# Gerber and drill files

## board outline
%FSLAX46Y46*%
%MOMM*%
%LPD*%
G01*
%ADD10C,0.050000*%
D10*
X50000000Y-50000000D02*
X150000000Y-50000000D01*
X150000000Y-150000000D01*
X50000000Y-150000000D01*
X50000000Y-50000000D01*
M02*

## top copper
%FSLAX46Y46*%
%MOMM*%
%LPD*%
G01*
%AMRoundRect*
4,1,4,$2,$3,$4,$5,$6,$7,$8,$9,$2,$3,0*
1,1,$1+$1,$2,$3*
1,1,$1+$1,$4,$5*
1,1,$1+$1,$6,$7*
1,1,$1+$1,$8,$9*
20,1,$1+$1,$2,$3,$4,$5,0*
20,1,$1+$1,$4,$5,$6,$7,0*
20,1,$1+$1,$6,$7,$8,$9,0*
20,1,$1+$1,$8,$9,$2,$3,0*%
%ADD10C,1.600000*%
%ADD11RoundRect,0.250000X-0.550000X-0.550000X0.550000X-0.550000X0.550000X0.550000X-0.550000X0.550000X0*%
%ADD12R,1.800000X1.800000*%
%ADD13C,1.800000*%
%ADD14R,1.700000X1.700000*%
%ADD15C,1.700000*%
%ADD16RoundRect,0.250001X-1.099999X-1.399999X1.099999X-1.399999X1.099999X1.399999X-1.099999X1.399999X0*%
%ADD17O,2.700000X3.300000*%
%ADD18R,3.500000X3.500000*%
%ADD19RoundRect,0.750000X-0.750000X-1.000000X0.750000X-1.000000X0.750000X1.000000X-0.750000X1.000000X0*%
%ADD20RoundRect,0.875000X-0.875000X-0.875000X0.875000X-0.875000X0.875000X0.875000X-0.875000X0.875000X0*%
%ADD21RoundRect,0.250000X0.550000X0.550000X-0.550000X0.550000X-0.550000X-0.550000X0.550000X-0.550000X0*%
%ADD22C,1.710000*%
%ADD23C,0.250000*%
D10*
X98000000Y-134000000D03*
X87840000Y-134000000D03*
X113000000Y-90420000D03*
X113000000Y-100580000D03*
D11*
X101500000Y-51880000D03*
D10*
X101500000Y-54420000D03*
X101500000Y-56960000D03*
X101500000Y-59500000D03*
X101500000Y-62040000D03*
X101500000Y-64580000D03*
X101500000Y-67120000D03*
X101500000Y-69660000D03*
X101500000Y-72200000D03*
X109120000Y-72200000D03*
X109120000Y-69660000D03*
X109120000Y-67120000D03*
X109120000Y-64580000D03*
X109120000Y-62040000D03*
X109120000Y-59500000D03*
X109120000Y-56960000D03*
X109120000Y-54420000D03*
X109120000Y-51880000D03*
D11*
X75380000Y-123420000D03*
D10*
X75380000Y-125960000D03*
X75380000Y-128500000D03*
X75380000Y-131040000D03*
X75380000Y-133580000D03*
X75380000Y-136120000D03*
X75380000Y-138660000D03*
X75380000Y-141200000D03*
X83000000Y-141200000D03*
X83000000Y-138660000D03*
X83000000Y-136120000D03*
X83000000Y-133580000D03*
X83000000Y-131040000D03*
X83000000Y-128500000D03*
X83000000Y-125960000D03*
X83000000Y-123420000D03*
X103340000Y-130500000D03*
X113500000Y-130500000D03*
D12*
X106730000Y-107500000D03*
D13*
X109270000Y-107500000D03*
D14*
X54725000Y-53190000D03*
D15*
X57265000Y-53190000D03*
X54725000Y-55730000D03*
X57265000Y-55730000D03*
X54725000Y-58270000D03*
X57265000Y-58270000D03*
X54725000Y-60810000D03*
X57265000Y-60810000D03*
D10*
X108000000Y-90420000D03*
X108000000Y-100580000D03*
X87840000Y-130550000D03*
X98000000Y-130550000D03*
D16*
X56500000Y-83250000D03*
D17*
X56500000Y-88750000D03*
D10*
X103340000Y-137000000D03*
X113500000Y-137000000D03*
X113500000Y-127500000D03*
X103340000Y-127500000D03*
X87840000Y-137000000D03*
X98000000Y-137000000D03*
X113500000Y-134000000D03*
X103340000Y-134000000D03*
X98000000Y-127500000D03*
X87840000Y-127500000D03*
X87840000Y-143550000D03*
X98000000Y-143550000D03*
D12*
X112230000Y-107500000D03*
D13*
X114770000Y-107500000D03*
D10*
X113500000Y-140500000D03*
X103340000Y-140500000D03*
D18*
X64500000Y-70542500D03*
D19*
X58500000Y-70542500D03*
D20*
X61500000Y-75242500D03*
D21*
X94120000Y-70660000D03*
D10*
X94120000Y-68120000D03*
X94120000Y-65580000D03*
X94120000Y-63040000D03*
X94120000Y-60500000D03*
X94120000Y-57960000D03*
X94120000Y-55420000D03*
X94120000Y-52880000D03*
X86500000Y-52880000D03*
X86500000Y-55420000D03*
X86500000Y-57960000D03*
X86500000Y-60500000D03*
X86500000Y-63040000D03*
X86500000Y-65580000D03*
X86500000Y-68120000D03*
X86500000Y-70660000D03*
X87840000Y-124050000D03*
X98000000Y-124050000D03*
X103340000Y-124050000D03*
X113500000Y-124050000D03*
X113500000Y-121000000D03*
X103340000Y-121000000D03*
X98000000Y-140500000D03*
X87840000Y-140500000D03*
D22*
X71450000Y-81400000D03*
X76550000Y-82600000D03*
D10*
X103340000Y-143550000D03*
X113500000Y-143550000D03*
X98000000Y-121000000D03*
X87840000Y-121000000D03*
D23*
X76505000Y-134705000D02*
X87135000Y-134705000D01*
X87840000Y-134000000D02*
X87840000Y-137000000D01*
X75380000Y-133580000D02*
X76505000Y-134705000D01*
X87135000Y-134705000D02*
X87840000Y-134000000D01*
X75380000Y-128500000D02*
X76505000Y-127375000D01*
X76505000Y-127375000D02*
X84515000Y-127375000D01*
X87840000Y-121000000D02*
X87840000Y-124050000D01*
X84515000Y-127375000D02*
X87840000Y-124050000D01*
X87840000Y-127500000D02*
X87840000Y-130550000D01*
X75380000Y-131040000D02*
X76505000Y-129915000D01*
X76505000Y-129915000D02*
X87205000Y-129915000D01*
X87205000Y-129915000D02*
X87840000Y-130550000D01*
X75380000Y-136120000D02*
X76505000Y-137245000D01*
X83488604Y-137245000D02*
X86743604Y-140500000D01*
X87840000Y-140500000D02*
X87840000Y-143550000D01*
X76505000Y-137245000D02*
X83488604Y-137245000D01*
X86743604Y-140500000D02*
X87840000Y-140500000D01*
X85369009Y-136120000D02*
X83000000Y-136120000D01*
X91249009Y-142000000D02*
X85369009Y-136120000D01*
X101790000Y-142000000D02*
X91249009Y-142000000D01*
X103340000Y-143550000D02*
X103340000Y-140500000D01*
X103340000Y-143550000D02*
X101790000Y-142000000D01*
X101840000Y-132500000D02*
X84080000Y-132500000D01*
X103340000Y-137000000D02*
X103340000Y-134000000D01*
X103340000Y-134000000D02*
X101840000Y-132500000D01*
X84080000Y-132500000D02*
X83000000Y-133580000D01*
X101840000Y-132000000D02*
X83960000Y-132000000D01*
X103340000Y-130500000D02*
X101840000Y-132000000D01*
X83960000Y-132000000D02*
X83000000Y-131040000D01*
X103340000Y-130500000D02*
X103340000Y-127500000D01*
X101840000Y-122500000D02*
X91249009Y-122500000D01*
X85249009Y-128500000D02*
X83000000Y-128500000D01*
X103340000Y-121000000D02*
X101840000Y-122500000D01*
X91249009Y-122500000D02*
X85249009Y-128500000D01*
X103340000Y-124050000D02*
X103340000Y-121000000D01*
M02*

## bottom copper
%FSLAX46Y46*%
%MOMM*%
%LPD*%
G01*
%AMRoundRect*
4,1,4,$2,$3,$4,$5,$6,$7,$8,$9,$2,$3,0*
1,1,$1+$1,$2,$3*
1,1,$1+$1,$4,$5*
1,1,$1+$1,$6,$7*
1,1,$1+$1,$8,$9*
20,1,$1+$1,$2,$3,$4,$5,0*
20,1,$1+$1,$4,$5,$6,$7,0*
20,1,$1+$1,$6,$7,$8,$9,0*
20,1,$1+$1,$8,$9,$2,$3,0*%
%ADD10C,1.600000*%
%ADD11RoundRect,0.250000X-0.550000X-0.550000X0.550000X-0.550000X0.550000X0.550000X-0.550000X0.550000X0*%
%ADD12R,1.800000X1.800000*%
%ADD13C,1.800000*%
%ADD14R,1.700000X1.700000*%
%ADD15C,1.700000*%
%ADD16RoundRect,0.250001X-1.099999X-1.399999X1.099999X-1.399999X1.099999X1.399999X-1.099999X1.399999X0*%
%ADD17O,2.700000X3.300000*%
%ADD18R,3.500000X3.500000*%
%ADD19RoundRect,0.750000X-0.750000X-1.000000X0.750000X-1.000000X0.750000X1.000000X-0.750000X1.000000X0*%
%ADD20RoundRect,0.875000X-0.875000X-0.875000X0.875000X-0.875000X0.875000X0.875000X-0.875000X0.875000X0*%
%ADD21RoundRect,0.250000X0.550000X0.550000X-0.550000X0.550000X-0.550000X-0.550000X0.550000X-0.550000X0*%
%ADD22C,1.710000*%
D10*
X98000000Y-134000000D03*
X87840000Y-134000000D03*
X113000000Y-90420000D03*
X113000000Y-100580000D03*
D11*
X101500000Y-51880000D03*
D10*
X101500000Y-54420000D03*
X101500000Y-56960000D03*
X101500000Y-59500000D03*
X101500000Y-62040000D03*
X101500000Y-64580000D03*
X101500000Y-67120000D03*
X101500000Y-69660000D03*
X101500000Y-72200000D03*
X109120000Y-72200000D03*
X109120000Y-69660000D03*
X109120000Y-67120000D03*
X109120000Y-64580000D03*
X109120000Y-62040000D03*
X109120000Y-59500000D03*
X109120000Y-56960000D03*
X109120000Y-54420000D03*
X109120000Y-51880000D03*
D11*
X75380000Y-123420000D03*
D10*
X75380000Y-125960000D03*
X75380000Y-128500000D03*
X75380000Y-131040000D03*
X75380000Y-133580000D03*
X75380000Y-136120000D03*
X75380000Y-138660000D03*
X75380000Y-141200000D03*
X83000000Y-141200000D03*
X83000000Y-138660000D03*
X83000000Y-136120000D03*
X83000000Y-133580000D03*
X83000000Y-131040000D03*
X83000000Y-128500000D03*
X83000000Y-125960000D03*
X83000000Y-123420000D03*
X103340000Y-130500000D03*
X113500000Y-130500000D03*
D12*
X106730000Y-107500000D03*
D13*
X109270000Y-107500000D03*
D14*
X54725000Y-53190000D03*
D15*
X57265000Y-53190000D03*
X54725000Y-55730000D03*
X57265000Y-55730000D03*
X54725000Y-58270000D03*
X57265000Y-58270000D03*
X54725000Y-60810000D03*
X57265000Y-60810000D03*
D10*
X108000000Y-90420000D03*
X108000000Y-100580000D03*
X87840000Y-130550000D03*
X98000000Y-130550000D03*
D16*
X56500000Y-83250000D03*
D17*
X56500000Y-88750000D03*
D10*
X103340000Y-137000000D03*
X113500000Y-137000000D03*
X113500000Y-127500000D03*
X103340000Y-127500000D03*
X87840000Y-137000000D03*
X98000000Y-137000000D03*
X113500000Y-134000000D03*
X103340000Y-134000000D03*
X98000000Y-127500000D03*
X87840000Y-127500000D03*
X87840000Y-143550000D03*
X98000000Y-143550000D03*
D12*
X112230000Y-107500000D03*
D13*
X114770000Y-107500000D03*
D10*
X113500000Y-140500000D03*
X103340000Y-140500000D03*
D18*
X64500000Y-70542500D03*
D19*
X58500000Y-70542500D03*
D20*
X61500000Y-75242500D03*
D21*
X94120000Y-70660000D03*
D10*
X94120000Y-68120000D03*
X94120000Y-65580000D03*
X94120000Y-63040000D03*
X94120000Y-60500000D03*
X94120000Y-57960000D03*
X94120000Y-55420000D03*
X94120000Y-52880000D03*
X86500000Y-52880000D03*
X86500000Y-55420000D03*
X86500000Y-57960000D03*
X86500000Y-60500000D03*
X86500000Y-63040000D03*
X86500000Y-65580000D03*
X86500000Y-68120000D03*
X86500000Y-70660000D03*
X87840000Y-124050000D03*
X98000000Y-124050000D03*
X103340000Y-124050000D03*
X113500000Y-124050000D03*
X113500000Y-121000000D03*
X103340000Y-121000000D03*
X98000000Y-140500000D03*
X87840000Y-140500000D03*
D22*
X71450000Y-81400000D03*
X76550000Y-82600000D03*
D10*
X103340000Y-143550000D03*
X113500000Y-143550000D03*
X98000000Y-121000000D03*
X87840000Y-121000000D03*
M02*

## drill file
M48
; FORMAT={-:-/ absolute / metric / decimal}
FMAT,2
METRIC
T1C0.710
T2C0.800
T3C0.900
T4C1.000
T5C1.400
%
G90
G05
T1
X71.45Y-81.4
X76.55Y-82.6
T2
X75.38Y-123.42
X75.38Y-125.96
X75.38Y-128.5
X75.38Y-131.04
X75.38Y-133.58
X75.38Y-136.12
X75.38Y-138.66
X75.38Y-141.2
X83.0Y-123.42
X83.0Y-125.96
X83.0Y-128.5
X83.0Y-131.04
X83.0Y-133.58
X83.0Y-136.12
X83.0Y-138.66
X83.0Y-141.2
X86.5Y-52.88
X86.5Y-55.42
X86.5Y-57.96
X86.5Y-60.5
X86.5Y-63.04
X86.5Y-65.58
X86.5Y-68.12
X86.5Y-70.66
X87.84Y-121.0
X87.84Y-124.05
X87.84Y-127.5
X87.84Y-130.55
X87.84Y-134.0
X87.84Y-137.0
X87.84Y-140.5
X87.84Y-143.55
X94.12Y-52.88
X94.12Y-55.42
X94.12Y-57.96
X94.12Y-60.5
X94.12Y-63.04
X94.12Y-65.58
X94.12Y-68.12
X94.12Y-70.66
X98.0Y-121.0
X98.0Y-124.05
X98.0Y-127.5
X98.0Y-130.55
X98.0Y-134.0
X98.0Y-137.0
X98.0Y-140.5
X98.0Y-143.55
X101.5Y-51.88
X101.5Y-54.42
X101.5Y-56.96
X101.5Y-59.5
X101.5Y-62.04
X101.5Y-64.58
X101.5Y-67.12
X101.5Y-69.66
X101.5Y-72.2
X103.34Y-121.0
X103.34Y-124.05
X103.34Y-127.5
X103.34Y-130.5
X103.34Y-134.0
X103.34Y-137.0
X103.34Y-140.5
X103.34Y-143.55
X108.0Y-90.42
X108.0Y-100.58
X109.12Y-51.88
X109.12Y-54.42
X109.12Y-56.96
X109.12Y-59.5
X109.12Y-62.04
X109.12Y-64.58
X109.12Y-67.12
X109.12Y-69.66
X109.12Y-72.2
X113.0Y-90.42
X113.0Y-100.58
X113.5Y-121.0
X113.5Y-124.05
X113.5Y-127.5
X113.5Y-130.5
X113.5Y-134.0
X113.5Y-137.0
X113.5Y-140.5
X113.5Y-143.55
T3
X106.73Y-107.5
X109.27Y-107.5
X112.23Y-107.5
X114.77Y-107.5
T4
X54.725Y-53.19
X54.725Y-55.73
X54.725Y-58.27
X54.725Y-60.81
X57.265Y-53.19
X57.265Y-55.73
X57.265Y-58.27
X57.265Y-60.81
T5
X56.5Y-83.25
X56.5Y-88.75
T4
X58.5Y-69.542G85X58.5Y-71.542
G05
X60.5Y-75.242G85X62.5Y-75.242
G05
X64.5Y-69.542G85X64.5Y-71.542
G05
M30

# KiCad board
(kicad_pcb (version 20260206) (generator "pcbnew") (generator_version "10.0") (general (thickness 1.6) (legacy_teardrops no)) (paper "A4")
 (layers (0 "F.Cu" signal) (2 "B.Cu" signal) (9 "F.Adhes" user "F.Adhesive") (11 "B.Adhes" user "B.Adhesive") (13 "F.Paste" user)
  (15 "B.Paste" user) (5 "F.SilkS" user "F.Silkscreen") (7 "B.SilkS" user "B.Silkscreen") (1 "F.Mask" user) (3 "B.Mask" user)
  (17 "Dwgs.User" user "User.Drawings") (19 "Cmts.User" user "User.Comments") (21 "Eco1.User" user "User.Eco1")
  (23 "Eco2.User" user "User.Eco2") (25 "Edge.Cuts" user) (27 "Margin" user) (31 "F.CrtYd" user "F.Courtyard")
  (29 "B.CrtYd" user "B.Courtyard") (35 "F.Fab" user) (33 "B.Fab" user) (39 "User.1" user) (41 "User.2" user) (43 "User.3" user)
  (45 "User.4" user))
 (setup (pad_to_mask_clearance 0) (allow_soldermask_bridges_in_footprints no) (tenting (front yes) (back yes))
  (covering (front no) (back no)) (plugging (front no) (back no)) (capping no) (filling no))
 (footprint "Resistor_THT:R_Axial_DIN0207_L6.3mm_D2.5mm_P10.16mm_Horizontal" (layer "F.Cu") (at 98 134 180)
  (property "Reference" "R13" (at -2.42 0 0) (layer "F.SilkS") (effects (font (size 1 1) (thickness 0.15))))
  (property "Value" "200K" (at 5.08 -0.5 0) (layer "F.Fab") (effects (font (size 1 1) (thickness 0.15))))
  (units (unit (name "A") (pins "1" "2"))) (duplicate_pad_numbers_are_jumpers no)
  (pad "1" thru_hole circle (at 0 0 180) (size 1.6 1.6) (drill 0.8) (layers "*.Cu" "*.Mask") (remove_unused_layers no) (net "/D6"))
  (pad "2" thru_hole circle (at 10.16 0 180) (size 1.6 1.6) (drill 0.8) (layers "*.Cu" "*.Mask") (remove_unused_layers no)
   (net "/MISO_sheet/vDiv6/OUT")))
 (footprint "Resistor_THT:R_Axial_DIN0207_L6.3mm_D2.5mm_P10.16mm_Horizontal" (layer "F.Cu") (at 113 90.42 -90)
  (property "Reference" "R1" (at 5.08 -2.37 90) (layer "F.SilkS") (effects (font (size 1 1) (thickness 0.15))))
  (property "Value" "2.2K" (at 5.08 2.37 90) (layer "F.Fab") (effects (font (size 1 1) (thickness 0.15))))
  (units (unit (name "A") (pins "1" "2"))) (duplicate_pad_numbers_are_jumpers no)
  (pad "1" thru_hole circle (at 0 0 270) (size 1.6 1.6) (drill 0.8) (layers "*.Cu" "*.Mask") (remove_unused_layers no) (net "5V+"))
  (pad "2" thru_hole circle (at 10.16 0 270) (size 1.6 1.6) (drill 0.8) (layers "*.Cu" "*.Mask") (remove_unused_layers no)
   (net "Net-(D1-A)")))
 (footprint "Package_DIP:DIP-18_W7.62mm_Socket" (layer "F.Cu") (at 101.5 51.88)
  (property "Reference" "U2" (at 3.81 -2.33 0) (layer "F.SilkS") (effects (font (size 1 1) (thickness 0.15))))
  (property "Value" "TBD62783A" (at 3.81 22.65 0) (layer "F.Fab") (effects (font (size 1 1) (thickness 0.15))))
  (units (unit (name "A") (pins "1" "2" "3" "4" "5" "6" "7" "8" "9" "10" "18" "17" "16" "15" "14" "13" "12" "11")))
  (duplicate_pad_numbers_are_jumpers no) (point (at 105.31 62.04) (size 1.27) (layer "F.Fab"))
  (pad "1" thru_hole roundrect (at 0 0) (size 1.6 1.6) (drill 0.8) (layers "*.Cu" "*.Mask") (remove_unused_layers no)
   (roundrect_rratio 0.15625) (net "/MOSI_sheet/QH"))
  (pad "2" thru_hole circle (at 0 2.54) (size 1.6 1.6) (drill 0.8) (layers "*.Cu" "*.Mask") (remove_unused_layers no) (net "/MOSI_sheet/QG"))
  (pad "3" thru_hole circle (at 0 5.08) (size 1.6 1.6) (drill 0.8) (layers "*.Cu" "*.Mask") (remove_unused_layers no) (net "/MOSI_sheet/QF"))
  (pad "4" thru_hole circle (at 0 7.62) (size 1.6 1.6) (drill 0.8) (layers "*.Cu" "*.Mask") (remove_unused_layers no) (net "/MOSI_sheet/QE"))
  (pad "5" thru_hole circle (at 0 10.16) (size 1.6 1.6) (drill 0.8) (layers "*.Cu" "*.Mask") (remove_unused_layers no)
   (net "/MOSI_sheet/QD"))
  (pad "6" thru_hole circle (at 0 12.7) (size 1.6 1.6) (drill 0.8) (layers "*.Cu" "*.Mask") (remove_unused_layers no) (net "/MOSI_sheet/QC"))
  (pad "7" thru_hole circle (at 0 15.24) (size 1.6 1.6) (drill 0.8) (layers "*.Cu" "*.Mask") (remove_unused_layers no)
   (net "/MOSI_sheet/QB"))
  (pad "8" thru_hole circle (at 0 17.78) (size 1.6 1.6) (drill 0.8) (layers "*.Cu" "*.Mask") (remove_unused_layers no)
   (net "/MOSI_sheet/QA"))
  (pad "9" thru_hole circle (at 0 20.32) (size 1.6 1.6) (drill 0.8) (layers "*.Cu" "*.Mask") (remove_unused_layers no) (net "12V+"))
  (pad "10" thru_hole circle (at 7.62 20.32) (size 1.6 1.6) (drill 0.8) (layers "*.Cu" "*.Mask") (remove_unused_layers no) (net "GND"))
  (pad "11" thru_hole circle (at 7.62 17.78) (size 1.6 1.6) (drill 0.8) (layers "*.Cu" "*.Mask") (remove_unused_layers no)
   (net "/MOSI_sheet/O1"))
  (pad "12" thru_hole circle (at 7.62 15.24) (size 1.6 1.6) (drill 0.8) (layers "*.Cu" "*.Mask") (remove_unused_layers no)
   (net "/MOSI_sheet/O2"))
  (pad "13" thru_hole circle (at 7.62 12.7) (size 1.6 1.6) (drill 0.8) (layers "*.Cu" "*.Mask") (remove_unused_layers no)
   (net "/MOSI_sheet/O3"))
  (pad "14" thru_hole circle (at 7.62 10.16) (size 1.6 1.6) (drill 0.8) (layers "*.Cu" "*.Mask") (remove_unused_layers no)
   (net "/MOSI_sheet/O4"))
  (pad "15" thru_hole circle (at 7.62 7.62) (size 1.6 1.6) (drill 0.8) (layers "*.Cu" "*.Mask") (remove_unused_layers no)
   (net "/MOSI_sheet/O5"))
  (pad "16" thru_hole circle (at 7.62 5.08) (size 1.6 1.6) (drill 0.8) (layers "*.Cu" "*.Mask") (remove_unused_layers no)
   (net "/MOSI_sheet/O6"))
  (pad "17" thru_hole circle (at 7.62 2.54) (size 1.6 1.6) (drill 0.8) (layers "*.Cu" "*.Mask") (remove_unused_layers no)
   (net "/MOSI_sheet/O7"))
  (pad "18" thru_hole circle (at 7.62 0) (size 1.6 1.6) (drill 0.8) (layers "*.Cu" "*.Mask") (remove_unused_layers no)
   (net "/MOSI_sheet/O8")))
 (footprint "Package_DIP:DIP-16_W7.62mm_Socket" (layer "F.Cu") (at 75.38 123.42)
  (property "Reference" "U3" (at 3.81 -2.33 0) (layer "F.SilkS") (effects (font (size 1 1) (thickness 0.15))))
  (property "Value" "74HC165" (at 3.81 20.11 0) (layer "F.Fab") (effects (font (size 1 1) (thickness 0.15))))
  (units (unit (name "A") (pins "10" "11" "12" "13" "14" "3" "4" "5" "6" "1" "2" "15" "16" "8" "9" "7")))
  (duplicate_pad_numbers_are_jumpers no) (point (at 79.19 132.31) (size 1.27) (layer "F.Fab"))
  (pad "1" thru_hole roundrect (at 0 0) (size 1.6 1.6) (drill 0.8) (layers "*.Cu" "*.Mask") (remove_unused_layers no)
   (roundrect_rratio 0.15625) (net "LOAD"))
  (pad "2" thru_hole circle (at 0 2.54) (size 1.6 1.6) (drill 0.8) (layers "*.Cu" "*.Mask") (remove_unused_layers no) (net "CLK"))
  (pad "3" thru_hole circle (at 0 5.08) (size 1.6 1.6) (drill 0.8) (layers "*.Cu" "*.Mask") (remove_unused_layers no)
   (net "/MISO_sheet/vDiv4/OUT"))
  (pad "4" thru_hole circle (at 0 7.62) (size 1.6 1.6) (drill 0.8) (layers "*.Cu" "*.Mask") (remove_unused_layers no)
   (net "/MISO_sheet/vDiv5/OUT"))
  (pad "5" thru_hole circle (at 0 10.16) (size 1.6 1.6) (drill 0.8) (layers "*.Cu" "*.Mask") (remove_unused_layers no)
   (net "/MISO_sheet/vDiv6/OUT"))
  (pad "6" thru_hole circle (at 0 12.7) (size 1.6 1.6) (drill 0.8) (layers "*.Cu" "*.Mask") (remove_unused_layers no)
   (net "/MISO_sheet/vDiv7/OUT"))
  (pad "7" thru_hole circle (at 0 15.24) (size 1.6 1.6) (drill 0.8) (layers "*.Cu" "*.Mask") (remove_unused_layers no)
   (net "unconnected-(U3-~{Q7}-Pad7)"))
  (pad "8" thru_hole circle (at 0 17.78) (size 1.6 1.6) (drill 0.8) (layers "*.Cu" "*.Mask") (remove_unused_layers no) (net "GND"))
  (pad "9" thru_hole circle (at 7.62 17.78) (size 1.6 1.6) (drill 0.8) (layers "*.Cu" "*.Mask") (remove_unused_layers no)
   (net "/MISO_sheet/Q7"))
  (pad "10" thru_hole circle (at 7.62 15.24) (size 1.6 1.6) (drill 0.8) (layers "*.Cu" "*.Mask") (remove_unused_layers no) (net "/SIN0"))
  (pad "11" thru_hole circle (at 7.62 12.7) (size 1.6 1.6) (drill 0.8) (layers "*.Cu" "*.Mask") (remove_unused_layers no)
   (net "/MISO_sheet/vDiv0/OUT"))
  (pad "12" thru_hole circle (at 7.62 10.16) (size 1.6 1.6) (drill 0.8) (layers "*.Cu" "*.Mask") (remove_unused_layers no)
   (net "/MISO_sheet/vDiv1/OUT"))
  (pad "13" thru_hole circle (at 7.62 7.62) (size 1.6 1.6) (drill 0.8) (layers "*.Cu" "*.Mask") (remove_unused_layers no)
   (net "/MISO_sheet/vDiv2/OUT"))
  (pad "14" thru_hole circle (at 7.62 5.08) (size 1.6 1.6) (drill 0.8) (layers "*.Cu" "*.Mask") (remove_unused_layers no)
   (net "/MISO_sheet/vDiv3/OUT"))
  (pad "15" thru_hole circle (at 7.62 2.54) (size 1.6 1.6) (drill 0.8) (layers "*.Cu" "*.Mask") (remove_unused_layers no) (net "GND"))
  (pad "16" thru_hole circle (at 7.62 0) (size 1.6 1.6) (drill 0.8) (layers "*.Cu" "*.Mask") (remove_unused_layers no)
   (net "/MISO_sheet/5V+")))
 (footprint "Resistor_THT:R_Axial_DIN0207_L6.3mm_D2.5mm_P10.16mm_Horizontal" (layer "F.Cu") (at 103.34 130.5)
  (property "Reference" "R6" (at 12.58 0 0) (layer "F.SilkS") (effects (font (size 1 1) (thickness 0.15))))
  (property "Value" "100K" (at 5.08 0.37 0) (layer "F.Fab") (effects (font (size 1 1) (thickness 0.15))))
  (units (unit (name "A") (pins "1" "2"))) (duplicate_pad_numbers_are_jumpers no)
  (pad "1" thru_hole circle (at 0 0) (size 1.6 1.6) (drill 0.8) (layers "*.Cu" "*.Mask") (remove_unused_layers no)
   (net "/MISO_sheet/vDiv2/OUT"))
  (pad "2" thru_hole circle (at 10.16 0) (size 1.6 1.6) (drill 0.8) (layers "*.Cu" "*.Mask") (remove_unused_layers no) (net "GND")))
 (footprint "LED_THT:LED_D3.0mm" (layer "F.Cu") (at 106.73 107.5)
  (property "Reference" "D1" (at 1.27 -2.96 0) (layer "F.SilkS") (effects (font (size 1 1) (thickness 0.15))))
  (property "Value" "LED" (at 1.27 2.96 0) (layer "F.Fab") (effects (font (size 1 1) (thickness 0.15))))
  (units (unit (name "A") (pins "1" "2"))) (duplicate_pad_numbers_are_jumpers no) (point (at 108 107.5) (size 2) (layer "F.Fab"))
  (pad "1" thru_hole rect (at 0 0) (size 1.8 1.8) (drill 0.9) (layers "*.Cu" "*.Mask") (remove_unused_layers no) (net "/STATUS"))
  (pad "2" thru_hole circle (at 2.54 0) (size 1.8 1.8) (drill 0.9) (layers "*.Cu" "*.Mask") (remove_unused_layers no) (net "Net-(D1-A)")))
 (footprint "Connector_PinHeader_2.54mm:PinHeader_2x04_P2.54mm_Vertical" (layer "F.Cu") (at 54.725 53.19)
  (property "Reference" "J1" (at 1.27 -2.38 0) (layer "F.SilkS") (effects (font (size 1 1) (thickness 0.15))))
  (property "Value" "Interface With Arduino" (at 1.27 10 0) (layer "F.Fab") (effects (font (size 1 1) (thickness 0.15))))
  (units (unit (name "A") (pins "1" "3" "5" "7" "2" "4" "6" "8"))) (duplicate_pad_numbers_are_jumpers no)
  (pad "1" thru_hole rect (at 0 0) (size 1.7 1.7) (drill 1) (layers "*.Cu" "*.Mask") (remove_unused_layers no) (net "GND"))
  (pad "2" thru_hole circle (at 2.54 0) (size 1.7 1.7) (drill 1) (layers "*.Cu" "*.Mask") (remove_unused_layers no) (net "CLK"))
  (pad "3" thru_hole circle (at 0 2.54) (size 1.7 1.7) (drill 1) (layers "*.Cu" "*.Mask") (remove_unused_layers no) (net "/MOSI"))
  (pad "4" thru_hole circle (at 2.54 2.54) (size 1.7 1.7) (drill 1) (layers "*.Cu" "*.Mask") (remove_unused_layers no) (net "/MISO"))
  (pad "5" thru_hole circle (at 0 5.08) (size 1.7 1.7) (drill 1) (layers "*.Cu" "*.Mask") (remove_unused_layers no) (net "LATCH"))
  (pad "6" thru_hole circle (at 2.54 5.08) (size 1.7 1.7) (drill 1) (layers "*.Cu" "*.Mask") (remove_unused_layers no) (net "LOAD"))
  (pad "7" thru_hole circle (at 0 7.62) (size 1.7 1.7) (drill 1) (layers "*.Cu" "*.Mask") (remove_unused_layers no) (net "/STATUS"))
  (pad "8" thru_hole circle (at 2.54 7.62) (size 1.7 1.7) (drill 1) (layers "*.Cu" "*.Mask") (remove_unused_layers no) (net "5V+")))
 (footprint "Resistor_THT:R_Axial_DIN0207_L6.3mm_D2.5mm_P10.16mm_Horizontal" (layer "F.Cu") (at 108 90.42 -90)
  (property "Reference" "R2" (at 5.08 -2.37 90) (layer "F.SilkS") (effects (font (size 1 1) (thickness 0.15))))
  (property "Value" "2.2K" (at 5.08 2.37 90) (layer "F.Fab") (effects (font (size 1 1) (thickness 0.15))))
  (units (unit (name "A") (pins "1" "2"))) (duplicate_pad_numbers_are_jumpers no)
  (pad "1" thru_hole circle (at 0 0 270) (size 1.6 1.6) (drill 0.8) (layers "*.Cu" "*.Mask") (remove_unused_layers no) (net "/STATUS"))
  (pad "2" thru_hole circle (at 10.16 0 270) (size 1.6 1.6) (drill 0.8) (layers "*.Cu" "*.Mask") (remove_unused_layers no)
   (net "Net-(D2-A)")))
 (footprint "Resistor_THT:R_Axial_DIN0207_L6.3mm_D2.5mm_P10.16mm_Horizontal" (layer "F.Cu") (at 87.84 130.55)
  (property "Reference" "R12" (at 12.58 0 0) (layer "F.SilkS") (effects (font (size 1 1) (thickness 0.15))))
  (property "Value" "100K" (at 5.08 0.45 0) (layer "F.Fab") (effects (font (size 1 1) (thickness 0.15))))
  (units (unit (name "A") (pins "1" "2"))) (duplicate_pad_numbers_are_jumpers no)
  (pad "1" thru_hole circle (at 0 0) (size 1.6 1.6) (drill 0.8) (layers "*.Cu" "*.Mask") (remove_unused_layers no)
   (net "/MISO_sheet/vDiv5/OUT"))
  (pad "2" thru_hole circle (at 10.16 0) (size 1.6 1.6) (drill 0.8) (layers "*.Cu" "*.Mask") (remove_unused_layers no) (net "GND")))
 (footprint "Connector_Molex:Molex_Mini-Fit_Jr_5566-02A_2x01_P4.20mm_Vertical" (layer "F.Cu") (at 56.5 83.25)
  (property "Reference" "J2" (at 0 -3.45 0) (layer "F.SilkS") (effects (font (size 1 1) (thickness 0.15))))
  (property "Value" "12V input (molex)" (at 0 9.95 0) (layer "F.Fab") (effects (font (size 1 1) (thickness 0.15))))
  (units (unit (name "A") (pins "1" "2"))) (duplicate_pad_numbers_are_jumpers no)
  (pad "1" thru_hole roundrect (at 0 0) (size 2.7 3.3) (drill 1.4) (layers "*.Cu" "*.Mask") (remove_unused_layers no)
   (roundrect_rratio 0.092593) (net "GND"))
  (pad "2" thru_hole oval (at 0 5.5) (size 2.7 3.3) (drill 1.4) (layers "*.Cu" "*.Mask") (remove_unused_layers no) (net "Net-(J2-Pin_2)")))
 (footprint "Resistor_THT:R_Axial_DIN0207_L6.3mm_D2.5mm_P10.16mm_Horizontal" (layer "F.Cu") (at 103.34 137)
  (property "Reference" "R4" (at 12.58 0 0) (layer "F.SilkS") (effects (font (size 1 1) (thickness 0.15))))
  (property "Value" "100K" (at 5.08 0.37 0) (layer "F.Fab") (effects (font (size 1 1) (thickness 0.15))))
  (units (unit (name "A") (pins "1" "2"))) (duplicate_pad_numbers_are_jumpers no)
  (pad "1" thru_hole circle (at 0 0) (size 1.6 1.6) (drill 0.8) (layers "*.Cu" "*.Mask") (remove_unused_layers no)
   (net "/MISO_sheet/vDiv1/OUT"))
  (pad "2" thru_hole circle (at 10.16 0) (size 1.6 1.6) (drill 0.8) (layers "*.Cu" "*.Mask") (remove_unused_layers no) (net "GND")))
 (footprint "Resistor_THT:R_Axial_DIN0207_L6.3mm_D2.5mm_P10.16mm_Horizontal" (layer "F.Cu") (at 113.5 127.5 180)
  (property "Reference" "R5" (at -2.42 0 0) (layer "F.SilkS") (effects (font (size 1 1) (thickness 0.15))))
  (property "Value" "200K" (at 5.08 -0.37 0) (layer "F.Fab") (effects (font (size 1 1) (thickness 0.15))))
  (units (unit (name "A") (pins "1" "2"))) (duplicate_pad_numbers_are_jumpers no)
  (pad "1" thru_hole circle (at 0 0 180) (size 1.6 1.6) (drill 0.8) (layers "*.Cu" "*.Mask") (remove_unused_layers no) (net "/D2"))
  (pad "2" thru_hole circle (at 10.16 0 180) (size 1.6 1.6) (drill 0.8) (layers "*.Cu" "*.Mask") (remove_unused_layers no)
   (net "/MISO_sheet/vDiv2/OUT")))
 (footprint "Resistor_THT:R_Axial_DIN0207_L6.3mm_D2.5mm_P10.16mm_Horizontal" (layer "F.Cu") (at 87.84 137)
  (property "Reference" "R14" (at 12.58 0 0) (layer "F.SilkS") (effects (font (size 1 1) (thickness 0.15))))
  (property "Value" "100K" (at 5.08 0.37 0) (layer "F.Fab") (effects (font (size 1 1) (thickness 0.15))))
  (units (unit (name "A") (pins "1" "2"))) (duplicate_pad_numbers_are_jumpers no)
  (pad "1" thru_hole circle (at 0 0) (size 1.6 1.6) (drill 0.8) (layers "*.Cu" "*.Mask") (remove_unused_layers no)
   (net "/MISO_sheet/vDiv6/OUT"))
  (pad "2" thru_hole circle (at 10.16 0) (size 1.6 1.6) (drill 0.8) (layers "*.Cu" "*.Mask") (remove_unused_layers no) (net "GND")))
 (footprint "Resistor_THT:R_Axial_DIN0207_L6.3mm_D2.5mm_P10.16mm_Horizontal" (layer "F.Cu") (at 113.5 134 180)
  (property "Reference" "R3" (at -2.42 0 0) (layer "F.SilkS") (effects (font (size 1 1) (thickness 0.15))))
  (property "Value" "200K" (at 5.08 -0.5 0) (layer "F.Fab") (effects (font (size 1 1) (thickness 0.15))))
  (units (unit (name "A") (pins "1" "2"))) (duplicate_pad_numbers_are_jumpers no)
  (pad "1" thru_hole circle (at 0 0 180) (size 1.6 1.6) (drill 0.8) (layers "*.Cu" "*.Mask") (remove_unused_layers no) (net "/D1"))
  (pad "2" thru_hole circle (at 10.16 0 180) (size 1.6 1.6) (drill 0.8) (layers "*.Cu" "*.Mask") (remove_unused_layers no)
   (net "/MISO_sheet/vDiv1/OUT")))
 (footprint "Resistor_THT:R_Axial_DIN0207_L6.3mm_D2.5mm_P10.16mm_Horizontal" (layer "F.Cu") (at 98 127.5 180)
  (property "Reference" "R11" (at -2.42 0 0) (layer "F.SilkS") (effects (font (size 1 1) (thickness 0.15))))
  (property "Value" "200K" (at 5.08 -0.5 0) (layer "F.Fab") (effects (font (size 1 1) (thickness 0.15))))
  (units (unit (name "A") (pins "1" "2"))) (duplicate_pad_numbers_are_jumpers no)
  (pad "1" thru_hole circle (at 0 0 180) (size 1.6 1.6) (drill 0.8) (layers "*.Cu" "*.Mask") (remove_unused_layers no) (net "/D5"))
  (pad "2" thru_hole circle (at 10.16 0 180) (size 1.6 1.6) (drill 0.8) (layers "*.Cu" "*.Mask") (remove_unused_layers no)
   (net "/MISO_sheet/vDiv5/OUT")))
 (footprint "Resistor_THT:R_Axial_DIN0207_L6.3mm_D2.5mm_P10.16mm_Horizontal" (layer "F.Cu") (at 87.84 143.55)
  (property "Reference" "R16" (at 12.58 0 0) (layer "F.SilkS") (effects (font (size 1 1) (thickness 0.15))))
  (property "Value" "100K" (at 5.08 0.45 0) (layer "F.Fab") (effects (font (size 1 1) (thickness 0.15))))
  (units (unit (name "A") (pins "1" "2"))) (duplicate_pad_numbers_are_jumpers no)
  (pad "1" thru_hole circle (at 0 0) (size 1.6 1.6) (drill 0.8) (layers "*.Cu" "*.Mask") (remove_unused_layers no)
   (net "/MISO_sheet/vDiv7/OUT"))
  (pad "2" thru_hole circle (at 10.16 0) (size 1.6 1.6) (drill 0.8) (layers "*.Cu" "*.Mask") (remove_unused_layers no) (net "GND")))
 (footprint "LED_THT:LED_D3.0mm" (layer "F.Cu") (at 112.23 107.5)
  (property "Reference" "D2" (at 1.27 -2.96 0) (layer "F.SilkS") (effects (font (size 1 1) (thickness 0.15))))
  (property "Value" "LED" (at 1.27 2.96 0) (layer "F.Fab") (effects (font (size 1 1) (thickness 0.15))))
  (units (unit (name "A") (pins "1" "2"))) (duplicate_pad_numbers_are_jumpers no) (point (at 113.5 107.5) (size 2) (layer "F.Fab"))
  (pad "1" thru_hole rect (at 0 0) (size 1.8 1.8) (drill 0.9) (layers "*.Cu" "*.Mask") (remove_unused_layers no) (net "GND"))
  (pad "2" thru_hole circle (at 2.54 0) (size 1.8 1.8) (drill 0.9) (layers "*.Cu" "*.Mask") (remove_unused_layers no) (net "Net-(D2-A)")))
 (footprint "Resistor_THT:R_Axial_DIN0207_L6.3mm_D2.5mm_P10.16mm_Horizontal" (layer "F.Cu") (at 113.5 140.5 180)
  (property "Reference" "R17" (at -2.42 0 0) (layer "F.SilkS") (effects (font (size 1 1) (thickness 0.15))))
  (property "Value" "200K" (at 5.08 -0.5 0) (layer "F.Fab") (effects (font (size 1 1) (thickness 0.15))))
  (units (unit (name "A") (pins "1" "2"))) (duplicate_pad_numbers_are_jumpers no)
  (pad "1" thru_hole circle (at 0 0 180) (size 1.6 1.6) (drill 0.8) (layers "*.Cu" "*.Mask") (remove_unused_layers no) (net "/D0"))
  (pad "2" thru_hole circle (at 10.16 0 180) (size 1.6 1.6) (drill 0.8) (layers "*.Cu" "*.Mask") (remove_unused_layers no)
   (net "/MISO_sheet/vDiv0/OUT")))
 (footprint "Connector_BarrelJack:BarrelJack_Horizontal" (layer "F.Cu") (at 64.5 70.5425)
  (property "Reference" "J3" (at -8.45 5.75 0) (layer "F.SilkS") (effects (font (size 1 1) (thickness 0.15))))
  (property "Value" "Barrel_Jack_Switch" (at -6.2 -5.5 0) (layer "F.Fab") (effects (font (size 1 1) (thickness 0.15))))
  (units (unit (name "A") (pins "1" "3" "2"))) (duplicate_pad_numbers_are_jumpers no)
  (pad "1" thru_hole rect (at 0 0) (size 3.5 3.5) (drill oval 1 3) (layers "*.Cu" "*.Mask") (remove_unused_layers no) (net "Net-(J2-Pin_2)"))
  (pad "2" thru_hole roundrect (at -6 0) (size 3 3.5) (drill oval 1 3) (layers "*.Cu" "*.Mask") (remove_unused_layers no)
   (roundrect_rratio 0.25) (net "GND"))
  (pad "3" thru_hole roundrect (at -3 4.7) (size 3.5 3.5) (drill oval 3 1) (layers "*.Cu" "*.Mask") (remove_unused_layers no)
   (roundrect_rratio 0.25) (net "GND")))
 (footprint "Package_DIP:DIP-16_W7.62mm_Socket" (layer "F.Cu") (at 94.12 70.66 180)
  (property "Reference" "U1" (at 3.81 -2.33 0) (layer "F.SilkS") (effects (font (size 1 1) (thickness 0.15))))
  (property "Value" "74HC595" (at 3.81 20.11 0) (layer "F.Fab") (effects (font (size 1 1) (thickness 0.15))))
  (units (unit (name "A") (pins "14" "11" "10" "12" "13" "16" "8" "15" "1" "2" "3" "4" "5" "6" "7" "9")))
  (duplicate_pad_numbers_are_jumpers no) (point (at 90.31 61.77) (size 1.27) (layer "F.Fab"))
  (pad "1" thru_hole roundrect (at 0 0 180) (size 1.6 1.6) (drill 0.8) (layers "*.Cu" "*.Mask") (remove_unused_layers no)
   (roundrect_rratio 0.15625) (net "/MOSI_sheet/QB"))
  (pad "2" thru_hole circle (at 0 2.54 180) (size 1.6 1.6) (drill 0.8) (layers "*.Cu" "*.Mask") (remove_unused_layers no)
   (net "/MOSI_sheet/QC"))
  (pad "3" thru_hole circle (at 0 5.08 180) (size 1.6 1.6) (drill 0.8) (layers "*.Cu" "*.Mask") (remove_unused_layers no)
   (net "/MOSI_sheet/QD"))
  (pad "4" thru_hole circle (at 0 7.62 180) (size 1.6 1.6) (drill 0.8) (layers "*.Cu" "*.Mask") (remove_unused_layers no)
   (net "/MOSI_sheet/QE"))
  (pad "5" thru_hole circle (at 0 10.16 180) (size 1.6 1.6) (drill 0.8) (layers "*.Cu" "*.Mask") (remove_unused_layers no)
   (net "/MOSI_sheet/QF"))
  (pad "6" thru_hole circle (at 0 12.7 180) (size 1.6 1.6) (drill 0.8) (layers "*.Cu" "*.Mask") (remove_unused_layers no)
   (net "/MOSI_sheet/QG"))
  (pad "7" thru_hole circle (at 0 15.24 180) (size 1.6 1.6) (drill 0.8) (layers "*.Cu" "*.Mask") (remove_unused_layers no)
   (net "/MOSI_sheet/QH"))
  (pad "8" thru_hole circle (at 0 17.78 180) (size 1.6 1.6) (drill 0.8) (layers "*.Cu" "*.Mask") (remove_unused_layers no) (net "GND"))
  (pad "9" thru_hole circle (at 7.62 17.78 180) (size 1.6 1.6) (drill 0.8) (layers "*.Cu" "*.Mask") (remove_unused_layers no)
   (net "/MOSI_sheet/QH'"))
  (pad "10" thru_hole circle (at 7.62 15.24 180) (size 1.6 1.6) (drill 0.8) (layers "*.Cu" "*.Mask") (remove_unused_layers no) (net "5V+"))
  (pad "11" thru_hole circle (at 7.62 12.7 180) (size 1.6 1.6) (drill 0.8) (layers "*.Cu" "*.Mask") (remove_unused_layers no) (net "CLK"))
  (pad "12" thru_hole circle (at 7.62 10.16 180) (size 1.6 1.6) (drill 0.8) (layers "*.Cu" "*.Mask") (remove_unused_layers no) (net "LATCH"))
  (pad "13" thru_hole circle (at 7.62 7.62 180) (size 1.6 1.6) (drill 0.8) (layers "*.Cu" "*.Mask") (remove_unused_layers no) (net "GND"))
  (pad "14" thru_hole circle (at 7.62 5.08 180) (size 1.6 1.6) (drill 0.8) (layers "*.Cu" "*.Mask") (remove_unused_layers no) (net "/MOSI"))
  (pad "15" thru_hole circle (at 7.62 2.54 180) (size 1.6 1.6) (drill 0.8) (layers "*.Cu" "*.Mask") (remove_unused_layers no)
   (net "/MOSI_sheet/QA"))
  (pad "16" thru_hole circle (at 7.62 0 180) (size 1.6 1.6) (drill 0.8) (layers "*.Cu" "*.Mask") (remove_unused_layers no) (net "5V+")))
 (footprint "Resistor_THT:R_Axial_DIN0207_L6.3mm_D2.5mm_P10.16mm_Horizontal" (layer "F.Cu") (at 87.84 124.05)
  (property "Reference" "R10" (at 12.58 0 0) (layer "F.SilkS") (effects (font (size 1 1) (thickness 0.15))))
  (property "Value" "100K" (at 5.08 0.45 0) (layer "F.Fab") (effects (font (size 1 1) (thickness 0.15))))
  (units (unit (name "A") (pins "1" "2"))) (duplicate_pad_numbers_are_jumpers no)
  (pad "1" thru_hole circle (at 0 0) (size 1.6 1.6) (drill 0.8) (layers "*.Cu" "*.Mask") (remove_unused_layers no)
   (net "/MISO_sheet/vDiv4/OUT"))
  (pad "2" thru_hole circle (at 10.16 0) (size 1.6 1.6) (drill 0.8) (layers "*.Cu" "*.Mask") (remove_unused_layers no) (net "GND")))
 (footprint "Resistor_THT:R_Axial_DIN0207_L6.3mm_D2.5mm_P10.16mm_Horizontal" (layer "F.Cu") (at 103.34 124.05)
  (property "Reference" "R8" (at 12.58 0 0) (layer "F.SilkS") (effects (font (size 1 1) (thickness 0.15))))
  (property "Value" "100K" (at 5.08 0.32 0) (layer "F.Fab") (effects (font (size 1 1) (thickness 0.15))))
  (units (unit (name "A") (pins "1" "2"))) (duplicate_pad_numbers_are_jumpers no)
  (pad "1" thru_hole circle (at 0 0) (size 1.6 1.6) (drill 0.8) (layers "*.Cu" "*.Mask") (remove_unused_layers no)
   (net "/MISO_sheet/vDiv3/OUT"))
  (pad "2" thru_hole circle (at 10.16 0) (size 1.6 1.6) (drill 0.8) (layers "*.Cu" "*.Mask") (remove_unused_layers no) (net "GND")))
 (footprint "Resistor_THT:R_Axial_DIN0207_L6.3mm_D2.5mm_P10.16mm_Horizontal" (layer "F.Cu") (at 113.5 121 180)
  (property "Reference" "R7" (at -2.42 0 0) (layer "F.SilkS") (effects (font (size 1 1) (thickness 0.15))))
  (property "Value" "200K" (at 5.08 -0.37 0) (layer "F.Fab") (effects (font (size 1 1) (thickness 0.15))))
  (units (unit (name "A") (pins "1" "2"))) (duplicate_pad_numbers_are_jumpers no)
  (pad "1" thru_hole circle (at 0 0 180) (size 1.6 1.6) (drill 0.8) (layers "*.Cu" "*.Mask") (remove_unused_layers no) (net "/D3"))
  (pad "2" thru_hole circle (at 10.16 0 180) (size 1.6 1.6) (drill 0.8) (layers "*.Cu" "*.Mask") (remove_unused_layers no)
   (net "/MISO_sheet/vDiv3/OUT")))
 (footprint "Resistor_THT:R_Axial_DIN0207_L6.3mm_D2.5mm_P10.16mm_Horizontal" (layer "F.Cu") (at 98 140.5 180)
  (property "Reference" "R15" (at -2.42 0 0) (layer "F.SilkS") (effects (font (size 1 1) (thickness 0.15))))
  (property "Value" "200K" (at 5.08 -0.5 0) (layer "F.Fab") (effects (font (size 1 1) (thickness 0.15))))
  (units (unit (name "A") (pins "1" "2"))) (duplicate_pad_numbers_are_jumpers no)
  (pad "1" thru_hole circle (at 0 0 180) (size 1.6 1.6) (drill 0.8) (layers "*.Cu" "*.Mask") (remove_unused_layers no) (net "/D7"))
  (pad "2" thru_hole circle (at 10.16 0 180) (size 1.6 1.6) (drill 0.8) (layers "*.Cu" "*.Mask") (remove_unused_layers no)
   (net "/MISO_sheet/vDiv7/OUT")))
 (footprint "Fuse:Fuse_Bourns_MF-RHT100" (layer "F.Cu") (at 71.45 81.4)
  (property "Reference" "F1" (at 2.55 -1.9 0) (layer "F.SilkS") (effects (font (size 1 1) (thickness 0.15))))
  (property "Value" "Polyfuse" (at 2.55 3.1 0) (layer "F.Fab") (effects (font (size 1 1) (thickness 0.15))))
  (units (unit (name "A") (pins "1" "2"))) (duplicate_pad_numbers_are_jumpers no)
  (pad "1" thru_hole circle (at 0 0) (size 1.71 1.71) (drill 0.71) (layers "*.Cu" "*.Mask") (remove_unused_layers no) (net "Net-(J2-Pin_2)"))
  (pad "2" thru_hole circle (at 5.1 1.2) (size 1.71 1.71) (drill 0.71) (layers "*.Cu" "*.Mask") (remove_unused_layers no) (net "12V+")))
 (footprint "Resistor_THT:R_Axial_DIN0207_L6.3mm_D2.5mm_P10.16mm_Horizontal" (layer "F.Cu") (at 103.34 143.55)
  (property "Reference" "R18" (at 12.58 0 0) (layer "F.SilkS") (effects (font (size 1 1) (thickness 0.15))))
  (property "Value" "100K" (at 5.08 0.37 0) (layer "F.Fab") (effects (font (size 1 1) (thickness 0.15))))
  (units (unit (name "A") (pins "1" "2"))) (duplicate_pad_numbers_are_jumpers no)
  (pad "1" thru_hole circle (at 0 0) (size 1.6 1.6) (drill 0.8) (layers "*.Cu" "*.Mask") (remove_unused_layers no)
   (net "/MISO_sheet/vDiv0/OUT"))
  (pad "2" thru_hole circle (at 10.16 0) (size 1.6 1.6) (drill 0.8) (layers "*.Cu" "*.Mask") (remove_unused_layers no) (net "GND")))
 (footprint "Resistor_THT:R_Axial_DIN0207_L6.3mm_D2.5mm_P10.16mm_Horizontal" (layer "F.Cu") (at 98 121 180)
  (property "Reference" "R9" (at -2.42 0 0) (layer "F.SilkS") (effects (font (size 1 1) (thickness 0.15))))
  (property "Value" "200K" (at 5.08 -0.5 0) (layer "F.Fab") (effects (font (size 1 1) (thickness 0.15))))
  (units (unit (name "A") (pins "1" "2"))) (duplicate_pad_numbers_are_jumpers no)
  (pad "1" thru_hole circle (at 0 0 180) (size 1.6 1.6) (drill 0.8) (layers "*.Cu" "*.Mask") (remove_unused_layers no) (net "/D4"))
  (pad "2" thru_hole circle (at 10.16 0 180) (size 1.6 1.6) (drill 0.8) (layers "*.Cu" "*.Mask") (remove_unused_layers no)
   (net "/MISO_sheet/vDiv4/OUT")))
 (gr_rect (start 50 50) (end 150 150) (stroke (width 0.05) (type solid)) (fill no) (layer "Edge.Cuts"))
 (segment (start 76.505 134.705) (end 87.135 134.705) (width 0.25) (layer "F.Cu") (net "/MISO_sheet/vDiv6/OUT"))
 (segment (start 87.84 134) (end 87.84 137) (width 0.25) (layer "F.Cu") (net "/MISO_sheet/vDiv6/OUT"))
 (segment (start 75.38 133.58) (end 76.505 134.705) (width 0.25) (layer "F.Cu") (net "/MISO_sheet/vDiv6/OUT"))
 (segment (start 87.135 134.705) (end 87.84 134) (width 0.25) (layer "F.Cu") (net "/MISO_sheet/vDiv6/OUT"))
 (segment (start 75.38 128.5) (end 76.505 127.375) (width 0.25) (layer "F.Cu") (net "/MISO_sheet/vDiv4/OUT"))
 (segment (start 76.505 127.375) (end 84.515 127.375) (width 0.25) (layer "F.Cu") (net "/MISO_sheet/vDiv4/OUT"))
 (segment (start 87.84 121) (end 87.84 124.05) (width 0.25) (layer "F.Cu") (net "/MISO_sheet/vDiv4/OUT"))
 (segment (start 84.515 127.375) (end 87.84 124.05) (width 0.25) (layer "F.Cu") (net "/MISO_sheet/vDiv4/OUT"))
 (segment (start 87.84 127.5) (end 87.84 130.55) (width 0.25) (layer "F.Cu") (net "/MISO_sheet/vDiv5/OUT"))
 (segment (start 75.38 131.04) (end 76.505 129.915) (width 0.25) (layer "F.Cu") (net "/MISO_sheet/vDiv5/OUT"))
 (segment (start 76.505 129.915) (end 87.205 129.915) (width 0.25) (layer "F.Cu") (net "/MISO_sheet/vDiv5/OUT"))
 (segment (start 87.205 129.915) (end 87.84 130.55) (width 0.25) (layer "F.Cu") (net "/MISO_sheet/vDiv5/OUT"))
 (segment (start 75.38 136.12) (end 76.505 137.245) (width 0.25) (layer "F.Cu") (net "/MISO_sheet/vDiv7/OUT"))
 (segment (start 83.488604 137.245) (end 86.743604 140.5) (width 0.25) (layer "F.Cu") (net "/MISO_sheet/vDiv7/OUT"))
 (segment (start 87.84 140.5) (end 87.84 143.55) (width 0.25) (layer "F.Cu") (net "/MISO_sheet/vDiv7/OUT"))
 (segment (start 76.505 137.245) (end 83.488604 137.245) (width 0.25) (layer "F.Cu") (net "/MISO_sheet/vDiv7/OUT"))
 (segment (start 86.743604 140.5) (end 87.84 140.5) (width 0.25) (layer "F.Cu") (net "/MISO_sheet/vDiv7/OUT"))
 (segment (start 85.369009 136.12) (end 83 136.12) (width 0.25) (layer "F.Cu") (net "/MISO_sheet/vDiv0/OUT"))
 (segment (start 91.249009 142) (end 85.369009 136.12) (width 0.25) (layer "F.Cu") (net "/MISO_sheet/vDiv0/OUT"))
 (segment (start 101.79 142) (end 91.249009 142) (width 0.25) (layer "F.Cu") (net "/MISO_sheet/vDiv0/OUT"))
 (segment (start 103.34 143.55) (end 103.34 140.5) (width 0.25) (layer "F.Cu") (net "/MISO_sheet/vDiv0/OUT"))
 (segment (start 103.34 143.55) (end 101.79 142) (width 0.25) (layer "F.Cu") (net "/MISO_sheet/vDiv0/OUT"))
 (segment (start 101.84 132.5) (end 84.08 132.5) (width 0.25) (layer "F.Cu") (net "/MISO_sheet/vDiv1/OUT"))
 (segment (start 103.34 137) (end 103.34 134) (width 0.25) (layer "F.Cu") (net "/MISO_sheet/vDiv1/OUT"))
 (segment (start 103.34 134) (end 101.84 132.5) (width 0.25) (layer "F.Cu") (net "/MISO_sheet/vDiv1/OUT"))
 (segment (start 84.08 132.5) (end 83 133.58) (width 0.25) (layer "F.Cu") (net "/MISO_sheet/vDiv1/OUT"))
 (segment (start 101.84 132) (end 83.96 132) (width 0.25) (layer "F.Cu") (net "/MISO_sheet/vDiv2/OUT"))
 (segment (start 103.34 130.5) (end 101.84 132) (width 0.25) (layer "F.Cu") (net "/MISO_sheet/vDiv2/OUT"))
 (segment (start 83.96 132) (end 83 131.04) (width 0.25) (layer "F.Cu") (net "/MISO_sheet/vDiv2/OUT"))
 (segment (start 103.34 130.5) (end 103.34 127.5) (width 0.25) (layer "F.Cu") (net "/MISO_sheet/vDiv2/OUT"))
 (segment (start 101.84 122.5) (end 91.249009 122.5) (width 0.25) (layer "F.Cu") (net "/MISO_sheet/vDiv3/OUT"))
 (segment (start 85.249009 128.5) (end 83 128.5) (width 0.25) (layer "F.Cu") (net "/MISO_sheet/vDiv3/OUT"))
 (segment (start 103.34 121) (end 101.84 122.5) (width 0.25) (layer "F.Cu") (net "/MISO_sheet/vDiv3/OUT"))
 (segment (start 91.249009 122.5) (end 85.249009 128.5) (width 0.25) (layer "F.Cu") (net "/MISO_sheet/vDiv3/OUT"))
 (segment (start 103.34 124.05) (end 103.34 121) (width 0.25) (layer "F.Cu") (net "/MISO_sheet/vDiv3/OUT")))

